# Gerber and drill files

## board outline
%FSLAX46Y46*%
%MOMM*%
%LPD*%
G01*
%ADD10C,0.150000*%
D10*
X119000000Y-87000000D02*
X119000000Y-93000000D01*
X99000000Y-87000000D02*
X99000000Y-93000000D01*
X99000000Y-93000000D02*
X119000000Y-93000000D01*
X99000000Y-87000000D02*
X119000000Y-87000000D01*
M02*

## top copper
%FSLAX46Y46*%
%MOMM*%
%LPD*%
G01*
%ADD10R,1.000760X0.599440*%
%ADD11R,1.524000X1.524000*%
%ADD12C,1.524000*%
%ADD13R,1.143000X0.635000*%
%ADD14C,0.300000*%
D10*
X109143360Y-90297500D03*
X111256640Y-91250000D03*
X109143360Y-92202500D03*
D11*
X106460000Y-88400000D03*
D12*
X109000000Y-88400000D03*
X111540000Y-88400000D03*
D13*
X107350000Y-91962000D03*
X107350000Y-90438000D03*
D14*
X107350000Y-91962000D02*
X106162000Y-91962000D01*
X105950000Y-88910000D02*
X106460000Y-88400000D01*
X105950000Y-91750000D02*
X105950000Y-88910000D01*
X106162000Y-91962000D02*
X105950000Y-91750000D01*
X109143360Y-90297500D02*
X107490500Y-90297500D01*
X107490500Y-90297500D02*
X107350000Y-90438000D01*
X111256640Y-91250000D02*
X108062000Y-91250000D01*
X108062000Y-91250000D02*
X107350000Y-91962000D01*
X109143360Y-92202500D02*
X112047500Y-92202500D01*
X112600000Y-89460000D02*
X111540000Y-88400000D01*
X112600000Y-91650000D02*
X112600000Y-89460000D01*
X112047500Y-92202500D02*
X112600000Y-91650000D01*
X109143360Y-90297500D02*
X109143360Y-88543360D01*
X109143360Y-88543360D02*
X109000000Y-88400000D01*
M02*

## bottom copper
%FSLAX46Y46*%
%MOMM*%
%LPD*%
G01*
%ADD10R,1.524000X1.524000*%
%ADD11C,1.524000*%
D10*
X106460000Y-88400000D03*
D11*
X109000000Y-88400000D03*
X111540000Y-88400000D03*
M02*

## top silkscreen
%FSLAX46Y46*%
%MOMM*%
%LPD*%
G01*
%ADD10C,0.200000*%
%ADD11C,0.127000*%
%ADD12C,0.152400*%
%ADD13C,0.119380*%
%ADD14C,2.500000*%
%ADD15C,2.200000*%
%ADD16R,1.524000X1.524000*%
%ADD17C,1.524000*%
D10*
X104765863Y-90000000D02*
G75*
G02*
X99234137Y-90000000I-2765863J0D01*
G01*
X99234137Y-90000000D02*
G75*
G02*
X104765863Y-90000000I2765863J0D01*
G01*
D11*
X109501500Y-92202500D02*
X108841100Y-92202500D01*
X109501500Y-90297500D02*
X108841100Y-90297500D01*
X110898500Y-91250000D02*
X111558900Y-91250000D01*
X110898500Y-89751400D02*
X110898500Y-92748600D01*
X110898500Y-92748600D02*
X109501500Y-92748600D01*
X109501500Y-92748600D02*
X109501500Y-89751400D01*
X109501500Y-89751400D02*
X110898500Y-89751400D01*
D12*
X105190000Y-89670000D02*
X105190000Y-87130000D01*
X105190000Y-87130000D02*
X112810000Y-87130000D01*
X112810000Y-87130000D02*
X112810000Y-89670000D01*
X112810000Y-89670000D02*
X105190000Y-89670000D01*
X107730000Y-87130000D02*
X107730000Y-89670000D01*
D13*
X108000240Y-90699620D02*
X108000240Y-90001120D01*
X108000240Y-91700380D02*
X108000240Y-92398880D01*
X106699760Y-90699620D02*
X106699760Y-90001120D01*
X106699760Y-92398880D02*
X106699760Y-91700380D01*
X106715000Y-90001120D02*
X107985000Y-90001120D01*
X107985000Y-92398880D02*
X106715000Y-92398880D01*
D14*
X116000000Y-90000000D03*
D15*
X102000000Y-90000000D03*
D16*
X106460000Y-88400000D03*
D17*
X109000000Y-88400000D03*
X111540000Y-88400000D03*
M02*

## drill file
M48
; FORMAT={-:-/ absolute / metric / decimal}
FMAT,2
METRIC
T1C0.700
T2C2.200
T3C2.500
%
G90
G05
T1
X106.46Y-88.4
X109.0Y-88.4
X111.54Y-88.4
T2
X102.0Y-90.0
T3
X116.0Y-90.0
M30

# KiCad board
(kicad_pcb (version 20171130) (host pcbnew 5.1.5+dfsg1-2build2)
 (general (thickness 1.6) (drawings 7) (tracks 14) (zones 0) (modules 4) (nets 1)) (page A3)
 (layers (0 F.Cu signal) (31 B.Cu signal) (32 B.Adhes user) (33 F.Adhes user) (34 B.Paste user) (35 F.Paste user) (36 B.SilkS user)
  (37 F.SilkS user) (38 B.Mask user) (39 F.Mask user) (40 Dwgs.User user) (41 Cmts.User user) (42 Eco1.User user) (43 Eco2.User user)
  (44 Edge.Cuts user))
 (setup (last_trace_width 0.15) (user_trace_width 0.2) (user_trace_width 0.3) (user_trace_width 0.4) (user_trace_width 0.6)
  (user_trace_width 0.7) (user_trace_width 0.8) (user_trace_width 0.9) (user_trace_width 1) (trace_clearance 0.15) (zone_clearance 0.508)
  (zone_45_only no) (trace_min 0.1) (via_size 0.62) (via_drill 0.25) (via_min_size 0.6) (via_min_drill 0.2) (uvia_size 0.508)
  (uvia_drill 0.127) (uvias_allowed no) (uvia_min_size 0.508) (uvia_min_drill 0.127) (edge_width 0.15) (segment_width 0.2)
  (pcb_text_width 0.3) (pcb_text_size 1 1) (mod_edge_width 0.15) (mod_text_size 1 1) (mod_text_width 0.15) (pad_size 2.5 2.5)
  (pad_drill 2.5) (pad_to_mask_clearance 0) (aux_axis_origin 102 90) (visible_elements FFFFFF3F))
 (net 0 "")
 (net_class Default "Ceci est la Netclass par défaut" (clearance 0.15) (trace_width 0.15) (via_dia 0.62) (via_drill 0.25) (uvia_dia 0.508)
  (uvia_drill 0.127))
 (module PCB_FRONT (layer F.Cu) (at 109 90)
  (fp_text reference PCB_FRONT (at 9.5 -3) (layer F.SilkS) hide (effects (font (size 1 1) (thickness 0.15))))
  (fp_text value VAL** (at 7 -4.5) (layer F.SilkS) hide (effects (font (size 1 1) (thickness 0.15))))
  (pad "" np_thru_hole circle (at 7 0) (size 2.5 2.5) (drill 2.5) (layers *.Cu *.Mask F.SilkS))
  (pad "" np_thru_hole circle (at -7 0) (size 2.2 2.2) (drill 2.2) (layers *.Cu *.Mask F.SilkS)))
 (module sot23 (layer F.Cu) (at 110.2 91.25 270)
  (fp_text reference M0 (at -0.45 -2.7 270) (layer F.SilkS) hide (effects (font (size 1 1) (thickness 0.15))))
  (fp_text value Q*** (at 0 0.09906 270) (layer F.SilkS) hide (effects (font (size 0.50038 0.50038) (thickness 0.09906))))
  (fp_line (start 0.9525 0.6985) (end 0.9525 1.3589) (layer F.SilkS) (width 0.127))
  (fp_line (start -0.9525 0.6985) (end -0.9525 1.3589) (layer F.SilkS) (width 0.127))
  (fp_line (start 0 -0.6985) (end 0 -1.3589) (layer F.SilkS) (width 0.127))
  (fp_line (start -1.4986 -0.6985) (end 1.4986 -0.6985) (layer F.SilkS) (width 0.127))
  (fp_line (start 1.4986 -0.6985) (end 1.4986 0.6985) (layer F.SilkS) (width 0.127))
  (fp_line (start 1.4986 0.6985) (end -1.4986 0.6985) (layer F.SilkS) (width 0.127))
  (fp_line (start -1.4986 0.6985) (end -1.4986 -0.6985) (layer F.SilkS) (width 0.127))
  (pad 1 smd rect (at -0.9525 1.05664 270) (size 0.59944 1.00076) (layers F.Cu F.Paste F.Mask))
  (pad 2 smd rect (at 0 -1.05664 270) (size 0.59944 1.00076) (layers F.Cu F.Paste F.Mask))
  (pad 3 smd rect (at 0.9525 1.05664 270) (size 0.59944 1.00076) (layers F.Cu F.Paste F.Mask)))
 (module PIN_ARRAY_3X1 (layer F.Cu) (at 109 88.4)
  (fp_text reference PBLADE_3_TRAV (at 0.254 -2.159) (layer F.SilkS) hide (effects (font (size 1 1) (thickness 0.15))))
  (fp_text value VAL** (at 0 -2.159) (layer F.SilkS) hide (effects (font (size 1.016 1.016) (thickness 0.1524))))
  (fp_line (start -3.81 1.27) (end -3.81 -1.27) (layer F.SilkS) (width 0.1524))
  (fp_line (start -3.81 -1.27) (end 3.81 -1.27) (layer F.SilkS) (width 0.1524))
  (fp_line (start 3.81 -1.27) (end 3.81 1.27) (layer F.SilkS) (width 0.1524))
  (fp_line (start 3.81 1.27) (end -3.81 1.27) (layer F.SilkS) (width 0.1524))
  (fp_line (start -1.27 -1.27) (end -1.27 1.27) (layer F.SilkS) (width 0.1524))
  (pad 1 thru_hole rect (at -2.54 0) (size 1.524 1.524) (drill 0.7) (layers *.Cu *.Mask F.SilkS))
  (pad 2 thru_hole circle (at 0 0) (size 1.524 1.524) (drill 0.7) (layers *.Cu *.Mask F.SilkS))
  (pad 3 thru_hole circle (at 2.54 0) (size 1.524 1.524) (drill 0.7) (layers *.Cu *.Mask F.SilkS)))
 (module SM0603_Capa (layer F.Cu) (at 107.35 91.2 90)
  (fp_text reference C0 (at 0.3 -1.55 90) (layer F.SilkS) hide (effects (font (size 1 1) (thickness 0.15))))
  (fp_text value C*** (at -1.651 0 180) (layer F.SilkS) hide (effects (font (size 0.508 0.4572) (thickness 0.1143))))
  (fp_line (start 0.50038 0.65024) (end 1.19888 0.65024) (layer F.SilkS) (width 0.11938))
  (fp_line (start -0.50038 0.65024) (end -1.19888 0.65024) (layer F.SilkS) (width 0.11938))
  (fp_line (start 0.50038 -0.65024) (end 1.19888 -0.65024) (layer F.SilkS) (width 0.11938))
  (fp_line (start -1.19888 -0.65024) (end -0.50038 -0.65024) (layer F.SilkS) (width 0.11938))
  (fp_line (start 1.19888 -0.635) (end 1.19888 0.635) (layer F.SilkS) (width 0.11938))
  (fp_line (start -1.19888 0.635) (end -1.19888 -0.635) (layer F.SilkS) (width 0.11938))
  (pad 1 smd rect (at -0.762 0 90) (size 0.635 1.143) (layers F.Cu F.Paste F.Mask))
  (pad 2 smd rect (at 0.762 0 90) (size 0.635 1.143) (layers F.Cu F.Paste F.Mask)))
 (gr_circle (center 102 90) (end 104.1 91.8) (layer F.SilkS) (width 0.2))
 (gr_line (start 119 87) (end 119 93) (angle 90) (layer Edge.Cuts) (width 0.15))
 (gr_line (start 99 87) (end 99 93) (angle 90) (layer Edge.Cuts) (width 0.15))
 (gr_line (start 99 93) (end 119 93) (angle 90) (layer Edge.Cuts) (width 0.15))
 (gr_line (start 99 87) (end 119 87) (angle 90) (layer Edge.Cuts) (width 0.15))
 (segment (start 107.35 91.962) (end 106.162 91.962) (width 0.3) (layer F.Cu) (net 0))
 (segment (start 105.95 88.91) (end 106.46 88.4) (width 0.3) (layer F.Cu) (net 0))
 (segment (start 105.95 91.75) (end 105.95 88.91) (width 0.3) (layer F.Cu) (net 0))
 (segment (start 106.162 91.962) (end 105.95 91.75) (width 0.3) (layer F.Cu) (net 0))
 (segment (start 109.14336 90.2975) (end 107.4905 90.2975) (width 0.3) (layer F.Cu) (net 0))
 (segment (start 107.4905 90.2975) (end 107.35 90.438) (width 0.3) (layer F.Cu) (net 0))
 (segment (start 111.25664 91.25) (end 108.062 91.25) (width 0.3) (layer F.Cu) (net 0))
 (segment (start 108.062 91.25) (end 107.35 91.962) (width 0.3) (layer F.Cu) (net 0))
 (segment (start 109.14336 92.2025) (end 112.0475 92.2025) (width 0.3) (layer F.Cu) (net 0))
 (segment (start 112.6 89.46) (end 111.54 88.4) (width 0.3) (layer F.Cu) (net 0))
 (segment (start 112.6 91.65) (end 112.6 89.46) (width 0.3) (layer F.Cu) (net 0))
 (segment (start 112.0475 92.2025) (end 112.6 91.65) (width 0.3) (layer F.Cu) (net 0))
 (segment (start 109.14336 90.2975) (end 109.14336 88.54336) (width 0.3) (layer F.Cu) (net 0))
 (segment (start 109.14336 88.54336) (end 109 88.4) (width 0.3) (layer F.Cu) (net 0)))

